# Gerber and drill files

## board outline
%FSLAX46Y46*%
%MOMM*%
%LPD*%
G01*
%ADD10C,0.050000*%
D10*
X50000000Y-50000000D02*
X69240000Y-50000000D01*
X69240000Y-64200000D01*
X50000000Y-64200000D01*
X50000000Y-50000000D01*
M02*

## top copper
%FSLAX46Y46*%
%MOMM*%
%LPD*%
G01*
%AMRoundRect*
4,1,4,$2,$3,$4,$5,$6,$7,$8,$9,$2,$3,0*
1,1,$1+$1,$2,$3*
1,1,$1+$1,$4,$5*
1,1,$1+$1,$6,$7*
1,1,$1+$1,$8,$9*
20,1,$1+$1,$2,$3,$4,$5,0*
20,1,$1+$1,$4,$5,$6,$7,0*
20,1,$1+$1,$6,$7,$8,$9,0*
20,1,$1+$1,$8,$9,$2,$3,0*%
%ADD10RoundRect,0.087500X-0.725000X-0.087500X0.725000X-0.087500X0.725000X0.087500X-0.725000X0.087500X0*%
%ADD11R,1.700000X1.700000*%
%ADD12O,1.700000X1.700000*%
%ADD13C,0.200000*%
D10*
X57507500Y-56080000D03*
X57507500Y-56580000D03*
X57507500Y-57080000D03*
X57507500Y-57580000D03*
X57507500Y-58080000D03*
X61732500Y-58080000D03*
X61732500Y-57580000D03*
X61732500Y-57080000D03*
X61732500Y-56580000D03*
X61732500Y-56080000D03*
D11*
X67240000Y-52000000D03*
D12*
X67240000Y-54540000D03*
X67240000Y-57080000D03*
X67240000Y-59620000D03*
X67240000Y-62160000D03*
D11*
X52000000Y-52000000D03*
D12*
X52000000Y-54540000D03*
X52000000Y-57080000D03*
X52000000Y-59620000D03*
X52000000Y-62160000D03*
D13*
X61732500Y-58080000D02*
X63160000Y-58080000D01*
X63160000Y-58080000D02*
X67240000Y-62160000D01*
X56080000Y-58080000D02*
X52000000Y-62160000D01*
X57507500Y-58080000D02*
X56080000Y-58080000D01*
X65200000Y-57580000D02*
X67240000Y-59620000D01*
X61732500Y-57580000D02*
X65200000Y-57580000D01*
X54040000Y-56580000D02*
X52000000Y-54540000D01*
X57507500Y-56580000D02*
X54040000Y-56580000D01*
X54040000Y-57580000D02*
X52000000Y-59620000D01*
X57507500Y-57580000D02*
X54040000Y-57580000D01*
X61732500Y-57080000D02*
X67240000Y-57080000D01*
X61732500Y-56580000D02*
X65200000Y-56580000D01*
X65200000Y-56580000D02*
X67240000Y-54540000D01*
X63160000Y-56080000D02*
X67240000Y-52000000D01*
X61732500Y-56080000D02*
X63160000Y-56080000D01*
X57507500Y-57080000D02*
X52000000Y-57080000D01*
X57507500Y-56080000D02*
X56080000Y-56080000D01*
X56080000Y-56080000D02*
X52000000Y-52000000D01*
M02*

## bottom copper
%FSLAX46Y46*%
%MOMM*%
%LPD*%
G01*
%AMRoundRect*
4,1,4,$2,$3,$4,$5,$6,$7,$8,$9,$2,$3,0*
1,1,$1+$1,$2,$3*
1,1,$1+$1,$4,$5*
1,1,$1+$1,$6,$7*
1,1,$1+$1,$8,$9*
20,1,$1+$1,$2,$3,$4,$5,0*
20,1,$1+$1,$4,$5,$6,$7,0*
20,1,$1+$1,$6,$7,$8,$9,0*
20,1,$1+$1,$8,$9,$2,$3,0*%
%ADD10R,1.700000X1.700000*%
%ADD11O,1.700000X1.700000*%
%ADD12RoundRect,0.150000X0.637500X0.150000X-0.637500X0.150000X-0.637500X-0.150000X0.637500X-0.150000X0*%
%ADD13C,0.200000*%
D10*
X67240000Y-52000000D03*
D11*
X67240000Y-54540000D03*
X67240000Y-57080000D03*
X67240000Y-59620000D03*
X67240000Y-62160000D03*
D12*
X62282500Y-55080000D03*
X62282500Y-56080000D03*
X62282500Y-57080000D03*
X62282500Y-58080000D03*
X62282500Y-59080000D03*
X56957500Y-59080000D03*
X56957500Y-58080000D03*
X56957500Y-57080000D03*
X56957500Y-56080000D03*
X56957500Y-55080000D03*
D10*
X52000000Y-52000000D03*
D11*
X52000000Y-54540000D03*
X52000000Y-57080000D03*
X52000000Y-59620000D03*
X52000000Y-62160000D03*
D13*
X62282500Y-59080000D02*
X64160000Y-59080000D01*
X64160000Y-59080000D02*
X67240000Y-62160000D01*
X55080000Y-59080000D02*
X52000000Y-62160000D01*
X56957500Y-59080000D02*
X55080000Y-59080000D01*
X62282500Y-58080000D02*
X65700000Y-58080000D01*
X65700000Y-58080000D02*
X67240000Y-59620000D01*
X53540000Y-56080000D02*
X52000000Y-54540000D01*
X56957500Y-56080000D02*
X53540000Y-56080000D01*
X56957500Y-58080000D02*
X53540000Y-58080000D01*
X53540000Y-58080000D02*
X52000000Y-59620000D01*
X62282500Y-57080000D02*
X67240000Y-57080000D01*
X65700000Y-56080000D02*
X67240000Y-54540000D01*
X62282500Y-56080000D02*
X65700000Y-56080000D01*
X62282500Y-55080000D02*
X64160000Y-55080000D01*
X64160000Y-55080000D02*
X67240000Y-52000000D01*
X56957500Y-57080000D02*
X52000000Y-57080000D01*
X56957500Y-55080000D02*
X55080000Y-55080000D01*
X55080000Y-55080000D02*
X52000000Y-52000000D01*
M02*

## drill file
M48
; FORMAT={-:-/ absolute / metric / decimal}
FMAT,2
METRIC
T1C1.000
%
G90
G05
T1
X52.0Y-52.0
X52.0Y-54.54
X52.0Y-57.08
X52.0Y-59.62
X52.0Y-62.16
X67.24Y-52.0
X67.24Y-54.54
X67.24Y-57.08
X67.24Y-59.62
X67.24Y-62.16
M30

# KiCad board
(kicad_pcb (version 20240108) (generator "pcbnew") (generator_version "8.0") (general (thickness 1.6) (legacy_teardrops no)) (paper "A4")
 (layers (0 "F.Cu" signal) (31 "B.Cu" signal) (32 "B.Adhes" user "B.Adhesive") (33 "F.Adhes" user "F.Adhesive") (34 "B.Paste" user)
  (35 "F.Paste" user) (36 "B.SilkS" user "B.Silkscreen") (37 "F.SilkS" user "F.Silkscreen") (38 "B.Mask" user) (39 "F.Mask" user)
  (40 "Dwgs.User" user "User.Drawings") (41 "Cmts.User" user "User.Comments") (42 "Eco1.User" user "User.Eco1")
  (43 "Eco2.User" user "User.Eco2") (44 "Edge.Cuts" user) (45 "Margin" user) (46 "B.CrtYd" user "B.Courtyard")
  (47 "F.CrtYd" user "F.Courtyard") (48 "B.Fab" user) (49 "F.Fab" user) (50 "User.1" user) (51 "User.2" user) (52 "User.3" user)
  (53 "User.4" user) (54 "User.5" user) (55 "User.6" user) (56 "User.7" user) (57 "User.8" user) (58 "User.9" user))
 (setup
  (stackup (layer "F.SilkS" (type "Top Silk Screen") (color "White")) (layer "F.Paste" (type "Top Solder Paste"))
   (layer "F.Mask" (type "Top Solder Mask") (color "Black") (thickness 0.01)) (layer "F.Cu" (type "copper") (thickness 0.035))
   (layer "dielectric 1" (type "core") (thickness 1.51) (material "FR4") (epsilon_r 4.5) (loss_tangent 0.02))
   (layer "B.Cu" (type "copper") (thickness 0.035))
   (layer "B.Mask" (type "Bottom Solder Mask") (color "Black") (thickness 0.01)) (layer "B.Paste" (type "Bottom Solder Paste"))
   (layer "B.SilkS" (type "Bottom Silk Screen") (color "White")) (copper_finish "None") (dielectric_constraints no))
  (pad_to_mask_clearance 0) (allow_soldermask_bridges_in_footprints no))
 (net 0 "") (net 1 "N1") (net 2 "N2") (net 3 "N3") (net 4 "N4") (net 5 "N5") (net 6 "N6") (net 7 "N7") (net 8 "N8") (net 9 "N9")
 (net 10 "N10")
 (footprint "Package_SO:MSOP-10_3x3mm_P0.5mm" (layer "F.Cu") (at 59.62 57.08)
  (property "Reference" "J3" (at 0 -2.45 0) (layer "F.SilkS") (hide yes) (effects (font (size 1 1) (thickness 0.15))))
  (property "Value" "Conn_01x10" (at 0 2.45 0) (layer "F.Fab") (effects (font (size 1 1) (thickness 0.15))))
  (pad "1" smd roundrect (at -2.1125 -1) (size 1.625 0.35) (layers "F.Cu" "F.Paste" "F.Mask") (roundrect_rratio 0.25) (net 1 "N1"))
  (pad "2" smd roundrect (at -2.1125 -0.5) (size 1.625 0.35) (layers "F.Cu" "F.Paste" "F.Mask") (roundrect_rratio 0.25) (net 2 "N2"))
  (pad "3" smd roundrect (at -2.1125 0) (size 1.625 0.35) (layers "F.Cu" "F.Paste" "F.Mask") (roundrect_rratio 0.25) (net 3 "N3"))
  (pad "4" smd roundrect (at -2.1125 0.5) (size 1.625 0.35) (layers "F.Cu" "F.Paste" "F.Mask") (roundrect_rratio 0.25) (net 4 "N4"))
  (pad "5" smd roundrect (at -2.1125 1) (size 1.625 0.35) (layers "F.Cu" "F.Paste" "F.Mask") (roundrect_rratio 0.25) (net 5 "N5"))
  (pad "6" smd roundrect (at 2.1125 1) (size 1.625 0.35) (layers "F.Cu" "F.Paste" "F.Mask") (roundrect_rratio 0.25) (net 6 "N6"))
  (pad "7" smd roundrect (at 2.1125 0.5) (size 1.625 0.35) (layers "F.Cu" "F.Paste" "F.Mask") (roundrect_rratio 0.25) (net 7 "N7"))
  (pad "8" smd roundrect (at 2.1125 0) (size 1.625 0.35) (layers "F.Cu" "F.Paste" "F.Mask") (roundrect_rratio 0.25) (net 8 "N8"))
  (pad "9" smd roundrect (at 2.1125 -0.5) (size 1.625 0.35) (layers "F.Cu" "F.Paste" "F.Mask") (roundrect_rratio 0.25) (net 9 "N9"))
  (pad "10" smd roundrect (at 2.1125 -1) (size 1.625 0.35) (layers "F.Cu" "F.Paste" "F.Mask") (roundrect_rratio 0.25) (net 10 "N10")))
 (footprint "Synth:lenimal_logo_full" (layer "F.Cu") (at 59.62 63)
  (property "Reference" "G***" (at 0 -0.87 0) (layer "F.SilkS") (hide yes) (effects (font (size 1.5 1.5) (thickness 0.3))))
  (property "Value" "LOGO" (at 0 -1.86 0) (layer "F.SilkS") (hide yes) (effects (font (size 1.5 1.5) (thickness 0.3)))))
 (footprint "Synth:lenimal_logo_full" (layer "B.Cu") (at 59.62 63 180)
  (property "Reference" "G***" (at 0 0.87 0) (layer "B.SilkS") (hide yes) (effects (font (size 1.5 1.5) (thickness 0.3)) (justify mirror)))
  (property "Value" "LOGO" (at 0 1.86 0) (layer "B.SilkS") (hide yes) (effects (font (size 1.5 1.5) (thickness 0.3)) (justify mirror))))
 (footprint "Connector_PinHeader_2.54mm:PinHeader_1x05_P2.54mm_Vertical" (layer "B.Cu") (at 67.24 52 180)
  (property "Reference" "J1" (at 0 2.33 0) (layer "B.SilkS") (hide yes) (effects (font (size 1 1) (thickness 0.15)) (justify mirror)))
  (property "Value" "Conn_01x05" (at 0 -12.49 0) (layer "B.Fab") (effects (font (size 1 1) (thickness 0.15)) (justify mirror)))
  (pad "1" thru_hole rect (at 0 0 180) (size 1.7 1.7) (drill 1) (layers "*.Cu" "*.Mask") (remove_unused_layers no) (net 10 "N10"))
  (pad "2" thru_hole oval (at 0 -2.54 180) (size 1.7 1.7) (drill 1) (layers "*.Cu" "*.Mask") (remove_unused_layers no) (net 9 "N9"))
  (pad "3" thru_hole oval (at 0 -5.08 180) (size 1.7 1.7) (drill 1) (layers "*.Cu" "*.Mask") (remove_unused_layers no) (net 8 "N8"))
  (pad "4" thru_hole oval (at 0 -7.62 180) (size 1.7 1.7) (drill 1) (layers "*.Cu" "*.Mask") (remove_unused_layers no) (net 7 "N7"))
  (pad "5" thru_hole oval (at 0 -10.16 180) (size 1.7 1.7) (drill 1) (layers "*.Cu" "*.Mask") (remove_unused_layers no) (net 6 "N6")))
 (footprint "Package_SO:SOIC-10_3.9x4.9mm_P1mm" (layer "B.Cu") (at 59.62 57.08 180)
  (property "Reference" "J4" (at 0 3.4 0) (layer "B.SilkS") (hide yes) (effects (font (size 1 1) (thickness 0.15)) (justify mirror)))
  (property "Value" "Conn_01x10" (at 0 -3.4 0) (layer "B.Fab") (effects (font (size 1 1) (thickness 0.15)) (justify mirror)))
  (pad "1" smd roundrect (at -2.6625 2 180) (size 1.575 0.6) (layers "B.Cu" "B.Paste" "B.Mask") (roundrect_rratio 0.25) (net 10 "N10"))
  (pad "2" smd roundrect (at -2.6625 1 180) (size 1.575 0.6) (layers "B.Cu" "B.Paste" "B.Mask") (roundrect_rratio 0.25) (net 9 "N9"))
  (pad "3" smd roundrect (at -2.6625 0 180) (size 1.575 0.6) (layers "B.Cu" "B.Paste" "B.Mask") (roundrect_rratio 0.25) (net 8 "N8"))
  (pad "4" smd roundrect (at -2.6625 -1 180) (size 1.575 0.6) (layers "B.Cu" "B.Paste" "B.Mask") (roundrect_rratio 0.25) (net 7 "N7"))
  (pad "5" smd roundrect (at -2.6625 -2 180) (size 1.575 0.6) (layers "B.Cu" "B.Paste" "B.Mask") (roundrect_rratio 0.25) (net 6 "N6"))
  (pad "6" smd roundrect (at 2.6625 -2 180) (size 1.575 0.6) (layers "B.Cu" "B.Paste" "B.Mask") (roundrect_rratio 0.25) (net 5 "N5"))
  (pad "7" smd roundrect (at 2.6625 -1 180) (size 1.575 0.6) (layers "B.Cu" "B.Paste" "B.Mask") (roundrect_rratio 0.25) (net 4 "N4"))
  (pad "8" smd roundrect (at 2.6625 0 180) (size 1.575 0.6) (layers "B.Cu" "B.Paste" "B.Mask") (roundrect_rratio 0.25) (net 3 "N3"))
  (pad "9" smd roundrect (at 2.6625 1 180) (size 1.575 0.6) (layers "B.Cu" "B.Paste" "B.Mask") (roundrect_rratio 0.25) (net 2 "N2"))
  (pad "10" smd roundrect (at 2.6625 2 180) (size 1.575 0.6) (layers "B.Cu" "B.Paste" "B.Mask") (roundrect_rratio 0.25) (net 1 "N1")))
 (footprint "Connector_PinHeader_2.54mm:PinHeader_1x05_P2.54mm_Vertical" (layer "B.Cu") (at 52 52 180)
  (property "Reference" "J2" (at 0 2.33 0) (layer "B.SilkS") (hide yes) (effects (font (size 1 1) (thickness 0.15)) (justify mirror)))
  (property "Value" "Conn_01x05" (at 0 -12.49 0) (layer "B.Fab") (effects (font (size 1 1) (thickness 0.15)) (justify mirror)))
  (pad "1" thru_hole rect (at 0 0 180) (size 1.7 1.7) (drill 1) (layers "*.Cu" "*.Mask") (remove_unused_layers no) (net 1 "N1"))
  (pad "2" thru_hole oval (at 0 -2.54 180) (size 1.7 1.7) (drill 1) (layers "*.Cu" "*.Mask") (remove_unused_layers no) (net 2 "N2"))
  (pad "3" thru_hole oval (at 0 -5.08 180) (size 1.7 1.7) (drill 1) (layers "*.Cu" "*.Mask") (remove_unused_layers no) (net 3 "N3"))
  (pad "4" thru_hole oval (at 0 -7.62 180) (size 1.7 1.7) (drill 1) (layers "*.Cu" "*.Mask") (remove_unused_layers no) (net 4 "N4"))
  (pad "5" thru_hole oval (at 0 -10.16 180) (size 1.7 1.7) (drill 1) (layers "*.Cu" "*.Mask") (remove_unused_layers no) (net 5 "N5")))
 (gr_rect (start 50 50) (end 69.24 64.2) (stroke (width 0.05) (type default)) (fill none) (layer "Edge.Cuts"))
 (segment (start 61.7325 58.08) (end 63.16 58.08) (width 0.2) (layer "F.Cu") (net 6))
 (segment (start 63.16 58.08) (end 67.24 62.16) (width 0.2) (layer "F.Cu") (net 6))
 (segment (start 62.2825 59.08) (end 64.16 59.08) (width 0.2) (layer "B.Cu") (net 6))
 (segment (start 64.16 59.08) (end 67.24 62.16) (width 0.2) (layer "B.Cu") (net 6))
 (segment (start 56.08 58.08) (end 52 62.16) (width 0.2) (layer "F.Cu") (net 5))
 (segment (start 57.5075 58.08) (end 56.08 58.08) (width 0.2) (layer "F.Cu") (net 5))
 (segment (start 55.08 59.08) (end 52 62.16) (width 0.2) (layer "B.Cu") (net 5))
 (segment (start 56.9575 59.08) (end 55.08 59.08) (width 0.2) (layer "B.Cu") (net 5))
 (segment (start 65.2 57.58) (end 67.24 59.62) (width 0.2) (layer "F.Cu") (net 7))
 (segment (start 61.7325 57.58) (end 65.2 57.58) (width 0.2) (layer "F.Cu") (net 7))
 (segment (start 62.2825 58.08) (end 65.7 58.08) (width 0.2) (layer "B.Cu") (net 7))
 (segment (start 65.7 58.08) (end 67.24 59.62) (width 0.2) (layer "B.Cu") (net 7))
 (segment (start 54.04 56.58) (end 52 54.54) (width 0.2) (layer "F.Cu") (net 2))
 (segment (start 57.5075 56.58) (end 54.04 56.58) (width 0.2) (layer "F.Cu") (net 2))
 (segment (start 53.54 56.08) (end 52 54.54) (width 0.2) (layer "B.Cu") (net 2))
 (segment (start 56.9575 56.08) (end 53.54 56.08) (width 0.2) (layer "B.Cu") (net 2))
 (segment (start 54.04 57.58) (end 52 59.62) (width 0.2) (layer "F.Cu") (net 4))
 (segment (start 57.5075 57.58) (end 54.04 57.58) (width 0.2) (layer "F.Cu") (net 4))
 (segment (start 56.9575 58.08) (end 53.54 58.08) (width 0.2) (layer "B.Cu") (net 4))
 (segment (start 53.54 58.08) (end 52 59.62) (width 0.2) (layer "B.Cu") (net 4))
 (segment (start 61.7325 57.08) (end 67.24 57.08) (width 0.2) (layer "F.Cu") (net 8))
 (segment (start 62.2825 57.08) (end 67.24 57.08) (width 0.2) (layer "B.Cu") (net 8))
 (segment (start 61.7325 56.58) (end 65.2 56.58) (width 0.2) (layer "F.Cu") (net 9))
 (segment (start 65.2 56.58) (end 67.24 54.54) (width 0.2) (layer "F.Cu") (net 9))
 (segment (start 65.7 56.08) (end 67.24 54.54) (width 0.2) (layer "B.Cu") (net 9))
 (segment (start 62.2825 56.08) (end 65.7 56.08) (width 0.2) (layer "B.Cu") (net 9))
 (segment (start 63.16 56.08) (end 67.24 52) (width 0.2) (layer "F.Cu") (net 10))
 (segment (start 61.7325 56.08) (end 63.16 56.08) (width 0.2) (layer "F.Cu") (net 10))
 (segment (start 62.2825 55.08) (end 64.16 55.08) (width 0.2) (layer "B.Cu") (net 10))
 (segment (start 64.16 55.08) (end 67.24 52) (width 0.2) (layer "B.Cu") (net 10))
 (segment (start 57.5075 57.08) (end 52 57.08) (width 0.2) (layer "F.Cu") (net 3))
 (segment (start 56.9575 57.08) (end 52 57.08) (width 0.2) (layer "B.Cu") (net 3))
 (segment (start 57.5075 56.08) (end 56.08 56.08) (width 0.2) (layer "F.Cu") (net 1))
 (segment (start 56.08 56.08) (end 52 52) (width 0.2) (layer "F.Cu") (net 1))
 (segment (start 56.9575 55.08) (end 55.08 55.08) (width 0.2) (layer "B.Cu") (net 1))
 (segment (start 55.08 55.08) (end 52 52) (width 0.2) (layer "B.Cu") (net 1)))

